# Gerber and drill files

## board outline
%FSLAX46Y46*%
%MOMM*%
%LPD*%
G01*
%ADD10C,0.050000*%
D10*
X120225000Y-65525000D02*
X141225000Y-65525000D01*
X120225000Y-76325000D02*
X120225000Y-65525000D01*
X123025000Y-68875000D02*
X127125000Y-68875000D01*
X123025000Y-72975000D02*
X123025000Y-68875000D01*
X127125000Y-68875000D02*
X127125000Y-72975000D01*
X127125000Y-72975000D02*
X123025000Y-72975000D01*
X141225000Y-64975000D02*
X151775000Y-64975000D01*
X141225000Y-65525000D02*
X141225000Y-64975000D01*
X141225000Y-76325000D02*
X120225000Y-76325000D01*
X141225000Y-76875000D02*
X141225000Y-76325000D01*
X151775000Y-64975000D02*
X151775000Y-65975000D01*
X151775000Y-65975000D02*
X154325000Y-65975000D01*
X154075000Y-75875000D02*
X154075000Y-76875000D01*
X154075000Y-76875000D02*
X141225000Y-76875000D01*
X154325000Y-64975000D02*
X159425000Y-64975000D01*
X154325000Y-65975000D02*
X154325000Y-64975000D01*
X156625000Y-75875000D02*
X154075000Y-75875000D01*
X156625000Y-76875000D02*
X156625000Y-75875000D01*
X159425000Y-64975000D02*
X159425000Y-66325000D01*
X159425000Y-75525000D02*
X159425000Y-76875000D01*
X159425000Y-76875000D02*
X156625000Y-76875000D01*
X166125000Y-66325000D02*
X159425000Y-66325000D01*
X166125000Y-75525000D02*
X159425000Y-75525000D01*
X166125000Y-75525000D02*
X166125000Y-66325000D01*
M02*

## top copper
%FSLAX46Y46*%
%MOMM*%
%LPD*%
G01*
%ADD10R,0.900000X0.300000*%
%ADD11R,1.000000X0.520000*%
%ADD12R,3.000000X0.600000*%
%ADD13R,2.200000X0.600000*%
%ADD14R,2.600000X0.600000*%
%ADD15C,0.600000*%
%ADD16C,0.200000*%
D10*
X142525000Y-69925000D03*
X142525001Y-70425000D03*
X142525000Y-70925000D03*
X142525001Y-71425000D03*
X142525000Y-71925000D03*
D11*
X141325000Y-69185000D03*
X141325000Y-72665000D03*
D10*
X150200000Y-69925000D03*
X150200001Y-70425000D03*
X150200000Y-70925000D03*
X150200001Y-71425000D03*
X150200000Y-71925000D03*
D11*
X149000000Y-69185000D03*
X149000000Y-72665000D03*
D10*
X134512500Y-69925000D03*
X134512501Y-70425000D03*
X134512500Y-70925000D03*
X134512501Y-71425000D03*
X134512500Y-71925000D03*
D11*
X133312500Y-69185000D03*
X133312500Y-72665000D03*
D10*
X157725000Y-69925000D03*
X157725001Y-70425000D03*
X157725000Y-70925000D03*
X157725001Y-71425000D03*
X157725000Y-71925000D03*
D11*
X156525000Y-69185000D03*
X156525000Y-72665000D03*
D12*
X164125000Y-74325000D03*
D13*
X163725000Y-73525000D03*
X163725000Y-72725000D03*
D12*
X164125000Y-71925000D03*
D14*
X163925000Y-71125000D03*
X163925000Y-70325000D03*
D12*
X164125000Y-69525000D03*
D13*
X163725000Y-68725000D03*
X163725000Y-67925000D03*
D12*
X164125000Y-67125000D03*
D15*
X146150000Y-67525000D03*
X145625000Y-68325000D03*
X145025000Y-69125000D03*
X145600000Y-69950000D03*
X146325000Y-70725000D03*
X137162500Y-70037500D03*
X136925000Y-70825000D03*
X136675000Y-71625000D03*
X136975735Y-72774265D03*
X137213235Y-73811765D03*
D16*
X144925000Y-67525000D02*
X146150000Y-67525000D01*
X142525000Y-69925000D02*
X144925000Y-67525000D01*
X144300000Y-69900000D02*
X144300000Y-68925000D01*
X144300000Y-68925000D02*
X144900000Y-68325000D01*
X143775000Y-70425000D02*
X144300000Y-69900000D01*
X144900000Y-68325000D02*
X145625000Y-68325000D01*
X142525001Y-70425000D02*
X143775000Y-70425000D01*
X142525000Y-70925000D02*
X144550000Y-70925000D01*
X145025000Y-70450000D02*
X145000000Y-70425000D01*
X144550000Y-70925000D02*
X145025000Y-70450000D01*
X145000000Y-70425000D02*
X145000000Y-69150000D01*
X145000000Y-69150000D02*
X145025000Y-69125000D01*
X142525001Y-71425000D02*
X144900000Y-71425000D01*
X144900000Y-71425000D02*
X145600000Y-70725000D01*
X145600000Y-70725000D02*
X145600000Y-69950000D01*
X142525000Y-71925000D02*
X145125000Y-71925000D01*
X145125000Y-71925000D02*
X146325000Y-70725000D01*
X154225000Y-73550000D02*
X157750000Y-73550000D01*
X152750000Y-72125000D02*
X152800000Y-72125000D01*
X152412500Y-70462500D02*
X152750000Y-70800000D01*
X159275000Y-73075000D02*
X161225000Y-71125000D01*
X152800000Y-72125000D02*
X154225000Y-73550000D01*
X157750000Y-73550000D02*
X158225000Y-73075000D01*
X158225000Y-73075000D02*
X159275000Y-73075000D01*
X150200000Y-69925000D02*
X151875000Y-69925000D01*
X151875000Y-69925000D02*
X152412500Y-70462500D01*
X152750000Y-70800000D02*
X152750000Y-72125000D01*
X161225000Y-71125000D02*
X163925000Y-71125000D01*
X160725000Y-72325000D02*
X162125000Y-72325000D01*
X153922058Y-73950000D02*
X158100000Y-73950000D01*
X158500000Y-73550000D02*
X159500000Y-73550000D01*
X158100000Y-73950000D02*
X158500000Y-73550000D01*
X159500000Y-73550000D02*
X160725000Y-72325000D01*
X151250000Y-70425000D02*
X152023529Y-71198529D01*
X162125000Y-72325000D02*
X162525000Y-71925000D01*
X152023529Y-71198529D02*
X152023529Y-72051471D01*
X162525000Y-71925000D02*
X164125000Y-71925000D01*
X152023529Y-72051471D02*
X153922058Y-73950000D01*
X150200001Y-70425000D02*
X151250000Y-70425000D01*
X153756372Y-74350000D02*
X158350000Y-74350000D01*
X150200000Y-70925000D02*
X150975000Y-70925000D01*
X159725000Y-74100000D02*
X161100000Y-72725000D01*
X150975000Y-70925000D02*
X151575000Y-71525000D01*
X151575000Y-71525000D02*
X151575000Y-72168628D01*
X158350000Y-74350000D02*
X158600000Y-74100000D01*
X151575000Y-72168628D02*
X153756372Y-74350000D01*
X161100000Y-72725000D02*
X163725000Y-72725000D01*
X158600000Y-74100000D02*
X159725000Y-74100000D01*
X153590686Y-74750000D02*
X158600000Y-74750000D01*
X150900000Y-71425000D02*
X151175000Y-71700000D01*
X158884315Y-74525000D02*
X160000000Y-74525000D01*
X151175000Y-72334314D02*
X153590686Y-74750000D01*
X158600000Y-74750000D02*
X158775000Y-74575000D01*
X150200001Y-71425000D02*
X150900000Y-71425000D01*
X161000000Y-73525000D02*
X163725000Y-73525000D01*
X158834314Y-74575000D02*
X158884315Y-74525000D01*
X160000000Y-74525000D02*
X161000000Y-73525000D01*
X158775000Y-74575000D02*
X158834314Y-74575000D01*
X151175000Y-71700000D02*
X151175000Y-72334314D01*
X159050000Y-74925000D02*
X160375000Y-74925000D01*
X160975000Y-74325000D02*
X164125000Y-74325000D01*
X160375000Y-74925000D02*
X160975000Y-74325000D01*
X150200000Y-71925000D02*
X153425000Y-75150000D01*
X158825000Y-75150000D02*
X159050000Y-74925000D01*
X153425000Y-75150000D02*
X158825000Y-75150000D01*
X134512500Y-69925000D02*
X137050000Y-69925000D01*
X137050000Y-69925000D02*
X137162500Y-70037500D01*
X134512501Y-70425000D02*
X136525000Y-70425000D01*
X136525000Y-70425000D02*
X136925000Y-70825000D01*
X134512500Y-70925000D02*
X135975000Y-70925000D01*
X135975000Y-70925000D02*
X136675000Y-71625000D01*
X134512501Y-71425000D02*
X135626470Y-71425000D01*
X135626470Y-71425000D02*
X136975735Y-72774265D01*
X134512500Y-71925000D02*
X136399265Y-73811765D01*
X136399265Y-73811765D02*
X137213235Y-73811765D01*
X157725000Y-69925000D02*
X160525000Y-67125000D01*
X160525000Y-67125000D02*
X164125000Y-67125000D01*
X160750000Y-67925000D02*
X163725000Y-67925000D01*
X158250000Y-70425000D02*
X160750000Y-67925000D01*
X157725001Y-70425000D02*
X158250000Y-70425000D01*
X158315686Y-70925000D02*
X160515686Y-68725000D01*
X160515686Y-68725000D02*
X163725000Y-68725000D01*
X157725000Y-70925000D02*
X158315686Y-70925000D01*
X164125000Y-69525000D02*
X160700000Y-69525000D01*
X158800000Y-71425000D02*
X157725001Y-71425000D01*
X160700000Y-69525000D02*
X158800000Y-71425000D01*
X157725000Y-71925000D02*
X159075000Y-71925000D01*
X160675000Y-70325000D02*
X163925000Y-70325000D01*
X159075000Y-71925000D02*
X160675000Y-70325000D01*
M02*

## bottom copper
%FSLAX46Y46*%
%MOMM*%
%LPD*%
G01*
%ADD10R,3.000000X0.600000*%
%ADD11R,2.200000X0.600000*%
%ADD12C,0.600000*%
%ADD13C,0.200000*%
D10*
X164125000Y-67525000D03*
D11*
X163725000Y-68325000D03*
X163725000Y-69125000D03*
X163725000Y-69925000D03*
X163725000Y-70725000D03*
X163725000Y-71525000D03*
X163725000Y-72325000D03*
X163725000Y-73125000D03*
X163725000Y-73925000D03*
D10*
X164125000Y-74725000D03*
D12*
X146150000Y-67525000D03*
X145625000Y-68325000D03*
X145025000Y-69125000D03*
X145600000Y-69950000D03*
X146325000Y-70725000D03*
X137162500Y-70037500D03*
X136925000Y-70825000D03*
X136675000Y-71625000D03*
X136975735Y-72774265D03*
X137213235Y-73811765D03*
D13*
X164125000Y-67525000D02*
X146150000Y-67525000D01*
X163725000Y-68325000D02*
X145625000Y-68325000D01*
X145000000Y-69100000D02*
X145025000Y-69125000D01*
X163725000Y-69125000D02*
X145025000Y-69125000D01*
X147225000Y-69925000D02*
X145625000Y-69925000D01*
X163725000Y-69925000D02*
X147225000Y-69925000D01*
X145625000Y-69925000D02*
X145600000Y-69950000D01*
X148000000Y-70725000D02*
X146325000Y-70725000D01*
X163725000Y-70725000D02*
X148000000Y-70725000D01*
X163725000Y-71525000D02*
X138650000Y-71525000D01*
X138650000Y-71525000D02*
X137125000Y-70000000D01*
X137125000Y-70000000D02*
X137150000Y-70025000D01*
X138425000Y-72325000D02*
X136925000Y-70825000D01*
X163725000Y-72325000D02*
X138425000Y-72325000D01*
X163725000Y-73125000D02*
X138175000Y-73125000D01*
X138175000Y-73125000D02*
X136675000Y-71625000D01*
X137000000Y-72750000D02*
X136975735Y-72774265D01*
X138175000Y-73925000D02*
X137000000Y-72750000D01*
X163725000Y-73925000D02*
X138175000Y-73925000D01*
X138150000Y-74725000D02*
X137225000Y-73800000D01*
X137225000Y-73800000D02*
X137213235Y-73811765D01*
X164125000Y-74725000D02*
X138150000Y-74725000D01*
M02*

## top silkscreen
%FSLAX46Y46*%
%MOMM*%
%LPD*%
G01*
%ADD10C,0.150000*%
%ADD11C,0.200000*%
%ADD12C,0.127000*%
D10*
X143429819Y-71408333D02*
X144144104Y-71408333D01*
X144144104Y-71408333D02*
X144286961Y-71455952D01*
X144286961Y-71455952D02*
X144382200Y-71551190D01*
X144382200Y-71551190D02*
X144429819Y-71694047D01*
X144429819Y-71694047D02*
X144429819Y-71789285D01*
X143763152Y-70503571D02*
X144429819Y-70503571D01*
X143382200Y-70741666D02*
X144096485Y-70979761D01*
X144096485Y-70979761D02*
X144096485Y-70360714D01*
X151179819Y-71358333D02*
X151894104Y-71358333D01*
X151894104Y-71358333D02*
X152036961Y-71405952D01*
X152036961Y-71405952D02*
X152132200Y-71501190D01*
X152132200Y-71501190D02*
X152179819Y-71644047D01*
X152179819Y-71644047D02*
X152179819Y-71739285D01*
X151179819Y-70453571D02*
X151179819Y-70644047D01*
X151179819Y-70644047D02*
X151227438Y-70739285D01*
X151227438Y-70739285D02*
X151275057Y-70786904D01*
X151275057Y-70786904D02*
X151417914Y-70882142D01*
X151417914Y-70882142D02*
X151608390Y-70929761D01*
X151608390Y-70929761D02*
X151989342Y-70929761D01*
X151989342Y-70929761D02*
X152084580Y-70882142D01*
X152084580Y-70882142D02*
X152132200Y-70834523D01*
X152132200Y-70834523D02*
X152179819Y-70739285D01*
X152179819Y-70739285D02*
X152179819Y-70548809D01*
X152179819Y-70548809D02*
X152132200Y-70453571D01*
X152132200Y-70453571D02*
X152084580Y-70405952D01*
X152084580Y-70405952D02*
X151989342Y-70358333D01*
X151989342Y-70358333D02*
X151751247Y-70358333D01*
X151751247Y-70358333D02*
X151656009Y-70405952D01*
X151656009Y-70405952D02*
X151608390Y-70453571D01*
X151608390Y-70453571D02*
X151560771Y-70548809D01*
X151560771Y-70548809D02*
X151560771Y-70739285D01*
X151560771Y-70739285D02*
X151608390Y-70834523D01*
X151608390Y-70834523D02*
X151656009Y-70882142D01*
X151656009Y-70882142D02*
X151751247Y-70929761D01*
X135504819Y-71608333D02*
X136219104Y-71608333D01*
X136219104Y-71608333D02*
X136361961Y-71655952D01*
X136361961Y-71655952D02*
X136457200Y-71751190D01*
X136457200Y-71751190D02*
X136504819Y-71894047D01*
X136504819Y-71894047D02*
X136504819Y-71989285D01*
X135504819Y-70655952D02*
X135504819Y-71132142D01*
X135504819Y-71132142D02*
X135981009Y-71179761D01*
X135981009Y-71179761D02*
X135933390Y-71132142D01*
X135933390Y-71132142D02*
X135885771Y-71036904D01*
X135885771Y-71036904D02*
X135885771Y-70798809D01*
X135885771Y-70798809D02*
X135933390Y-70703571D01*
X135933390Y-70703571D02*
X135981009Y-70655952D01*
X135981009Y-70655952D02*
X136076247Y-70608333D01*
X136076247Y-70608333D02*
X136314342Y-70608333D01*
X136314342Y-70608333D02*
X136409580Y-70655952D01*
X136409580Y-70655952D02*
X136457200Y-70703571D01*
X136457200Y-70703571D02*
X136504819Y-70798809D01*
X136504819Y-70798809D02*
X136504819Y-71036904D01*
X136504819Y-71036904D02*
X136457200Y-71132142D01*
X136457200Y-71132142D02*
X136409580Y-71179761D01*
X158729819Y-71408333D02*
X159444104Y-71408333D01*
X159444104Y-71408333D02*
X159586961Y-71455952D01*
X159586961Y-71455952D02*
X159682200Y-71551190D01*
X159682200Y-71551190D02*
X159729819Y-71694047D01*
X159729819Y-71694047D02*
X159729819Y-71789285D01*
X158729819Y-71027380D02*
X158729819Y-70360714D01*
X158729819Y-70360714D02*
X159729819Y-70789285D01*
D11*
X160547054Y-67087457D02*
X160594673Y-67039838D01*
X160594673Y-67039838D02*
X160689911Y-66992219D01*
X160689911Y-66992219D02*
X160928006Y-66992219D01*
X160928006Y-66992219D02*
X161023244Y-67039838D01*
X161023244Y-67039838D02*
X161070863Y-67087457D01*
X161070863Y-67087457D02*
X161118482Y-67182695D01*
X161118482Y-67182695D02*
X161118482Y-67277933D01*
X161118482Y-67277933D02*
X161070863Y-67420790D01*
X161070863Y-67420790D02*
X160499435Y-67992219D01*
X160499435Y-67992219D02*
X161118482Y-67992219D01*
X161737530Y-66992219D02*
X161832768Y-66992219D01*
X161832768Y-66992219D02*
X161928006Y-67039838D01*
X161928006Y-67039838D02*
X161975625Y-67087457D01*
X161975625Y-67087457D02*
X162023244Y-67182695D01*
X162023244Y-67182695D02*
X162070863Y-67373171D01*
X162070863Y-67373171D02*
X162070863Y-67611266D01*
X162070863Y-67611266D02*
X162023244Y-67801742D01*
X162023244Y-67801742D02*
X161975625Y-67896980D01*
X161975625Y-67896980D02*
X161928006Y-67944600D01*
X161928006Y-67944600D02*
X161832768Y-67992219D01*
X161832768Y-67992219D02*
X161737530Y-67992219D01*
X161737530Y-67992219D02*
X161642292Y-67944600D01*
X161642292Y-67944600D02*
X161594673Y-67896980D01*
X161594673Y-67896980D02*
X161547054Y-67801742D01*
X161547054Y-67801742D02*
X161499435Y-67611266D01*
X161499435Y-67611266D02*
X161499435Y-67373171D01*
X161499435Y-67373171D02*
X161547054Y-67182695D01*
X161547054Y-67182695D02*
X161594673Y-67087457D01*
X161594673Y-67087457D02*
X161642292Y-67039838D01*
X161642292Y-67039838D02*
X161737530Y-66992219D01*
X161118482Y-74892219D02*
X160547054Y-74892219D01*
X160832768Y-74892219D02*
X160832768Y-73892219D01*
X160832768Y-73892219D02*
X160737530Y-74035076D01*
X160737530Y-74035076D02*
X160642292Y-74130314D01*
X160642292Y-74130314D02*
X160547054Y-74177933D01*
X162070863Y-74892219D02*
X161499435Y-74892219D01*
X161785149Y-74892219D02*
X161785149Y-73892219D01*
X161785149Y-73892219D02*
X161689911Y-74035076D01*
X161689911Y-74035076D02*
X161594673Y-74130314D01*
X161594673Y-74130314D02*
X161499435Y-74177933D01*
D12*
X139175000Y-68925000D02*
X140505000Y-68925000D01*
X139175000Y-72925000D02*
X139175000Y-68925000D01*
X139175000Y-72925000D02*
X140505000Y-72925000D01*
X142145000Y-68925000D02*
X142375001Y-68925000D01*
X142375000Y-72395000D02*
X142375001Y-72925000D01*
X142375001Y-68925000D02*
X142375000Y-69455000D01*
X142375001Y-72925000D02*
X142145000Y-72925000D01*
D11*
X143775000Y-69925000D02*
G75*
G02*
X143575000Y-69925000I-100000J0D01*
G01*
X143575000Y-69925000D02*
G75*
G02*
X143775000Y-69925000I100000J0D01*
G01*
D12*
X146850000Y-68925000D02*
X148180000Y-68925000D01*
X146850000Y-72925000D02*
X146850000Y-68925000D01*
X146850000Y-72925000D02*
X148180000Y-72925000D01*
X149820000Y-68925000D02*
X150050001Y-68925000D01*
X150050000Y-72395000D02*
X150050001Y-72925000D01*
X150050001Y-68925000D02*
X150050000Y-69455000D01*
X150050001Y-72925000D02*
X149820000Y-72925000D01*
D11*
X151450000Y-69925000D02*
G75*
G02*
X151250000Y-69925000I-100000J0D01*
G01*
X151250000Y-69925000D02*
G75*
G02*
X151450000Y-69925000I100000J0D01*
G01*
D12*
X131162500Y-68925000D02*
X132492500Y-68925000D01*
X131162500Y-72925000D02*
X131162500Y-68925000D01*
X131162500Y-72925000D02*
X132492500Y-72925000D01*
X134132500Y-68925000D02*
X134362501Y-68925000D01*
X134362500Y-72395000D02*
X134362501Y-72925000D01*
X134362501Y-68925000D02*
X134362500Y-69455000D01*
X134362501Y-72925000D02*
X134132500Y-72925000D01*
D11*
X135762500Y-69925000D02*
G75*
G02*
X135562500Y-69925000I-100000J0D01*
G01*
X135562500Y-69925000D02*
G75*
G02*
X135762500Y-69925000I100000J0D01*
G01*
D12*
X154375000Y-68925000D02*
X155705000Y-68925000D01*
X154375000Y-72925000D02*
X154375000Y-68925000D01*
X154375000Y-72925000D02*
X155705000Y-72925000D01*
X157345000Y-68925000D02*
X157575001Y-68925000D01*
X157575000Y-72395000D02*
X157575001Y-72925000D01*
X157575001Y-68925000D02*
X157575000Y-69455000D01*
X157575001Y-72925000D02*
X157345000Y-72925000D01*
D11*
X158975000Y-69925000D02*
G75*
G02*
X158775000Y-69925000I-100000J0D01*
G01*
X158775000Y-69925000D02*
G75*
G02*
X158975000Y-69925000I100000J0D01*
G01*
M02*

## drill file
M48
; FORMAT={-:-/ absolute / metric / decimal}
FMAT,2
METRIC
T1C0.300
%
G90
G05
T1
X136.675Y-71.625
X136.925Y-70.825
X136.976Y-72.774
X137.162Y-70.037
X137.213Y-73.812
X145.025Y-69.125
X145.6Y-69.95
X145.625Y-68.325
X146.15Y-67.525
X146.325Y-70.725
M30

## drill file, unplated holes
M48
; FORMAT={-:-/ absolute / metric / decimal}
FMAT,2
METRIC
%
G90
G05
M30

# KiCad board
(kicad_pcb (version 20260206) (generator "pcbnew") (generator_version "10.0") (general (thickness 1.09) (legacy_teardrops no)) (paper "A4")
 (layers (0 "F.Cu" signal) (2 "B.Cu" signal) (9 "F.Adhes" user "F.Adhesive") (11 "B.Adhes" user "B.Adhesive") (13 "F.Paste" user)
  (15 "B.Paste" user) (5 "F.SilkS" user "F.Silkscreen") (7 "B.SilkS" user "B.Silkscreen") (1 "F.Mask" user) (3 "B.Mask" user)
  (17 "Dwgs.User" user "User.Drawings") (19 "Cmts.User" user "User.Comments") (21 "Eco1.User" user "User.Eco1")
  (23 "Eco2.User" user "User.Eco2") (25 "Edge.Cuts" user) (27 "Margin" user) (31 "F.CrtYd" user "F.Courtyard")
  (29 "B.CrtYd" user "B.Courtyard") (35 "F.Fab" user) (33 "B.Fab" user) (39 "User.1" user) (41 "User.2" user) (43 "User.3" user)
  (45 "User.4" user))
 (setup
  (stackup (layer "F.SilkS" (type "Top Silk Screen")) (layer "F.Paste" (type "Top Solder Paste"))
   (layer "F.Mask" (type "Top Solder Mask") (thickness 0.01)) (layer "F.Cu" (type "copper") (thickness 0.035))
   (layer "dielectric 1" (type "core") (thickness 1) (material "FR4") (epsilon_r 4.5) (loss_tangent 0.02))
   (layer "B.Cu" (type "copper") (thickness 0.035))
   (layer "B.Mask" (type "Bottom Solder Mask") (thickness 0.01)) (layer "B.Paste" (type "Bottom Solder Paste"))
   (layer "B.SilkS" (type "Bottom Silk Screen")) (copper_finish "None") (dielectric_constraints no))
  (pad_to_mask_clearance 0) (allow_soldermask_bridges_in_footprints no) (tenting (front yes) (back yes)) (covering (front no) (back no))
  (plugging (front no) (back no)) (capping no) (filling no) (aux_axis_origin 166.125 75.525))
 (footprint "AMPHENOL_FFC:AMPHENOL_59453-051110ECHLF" (layer "F.Cu") (at 141.325 70.925 -90)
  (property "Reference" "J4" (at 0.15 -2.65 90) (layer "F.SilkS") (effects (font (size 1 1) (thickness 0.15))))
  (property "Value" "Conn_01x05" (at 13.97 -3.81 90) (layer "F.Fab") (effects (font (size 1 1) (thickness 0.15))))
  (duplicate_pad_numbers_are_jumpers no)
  (fp_line (start -2 2.15) (end -2 0.82) (stroke (width 0.127) (type solid)) (layer "F.SilkS"))
  (fp_line (start 2 2.15) (end -2 2.15) (stroke (width 0.127) (type solid)) (layer "F.SilkS"))
  (fp_line (start 2 2.15) (end 2 0.82) (stroke (width 0.127) (type solid)) (layer "F.SilkS"))
  (fp_line (start -2 -0.82) (end -2 -1.050001) (stroke (width 0.127) (type solid)) (layer "F.SilkS"))
  (fp_line (start 1.47 -1.05) (end 2 -1.050001) (stroke (width 0.127) (type solid)) (layer "F.SilkS"))
  (fp_line (start -2 -1.050001) (end -1.47 -1.05) (stroke (width 0.127) (type solid)) (layer "F.SilkS"))
  (fp_line (start 2 -1.050001) (end 2 -0.82) (stroke (width 0.127) (type solid)) (layer "F.SilkS"))
  (fp_circle (center -1 -2.35) (end -0.9 -2.35) (stroke (width 0.2) (type solid)) (fill no) (layer "F.SilkS"))
  (pad "1" smd rect (at -1 -1.2 270) (size 0.3 0.9) (layers "F.Cu" "F.Mask" "F.Paste") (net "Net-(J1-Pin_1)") (solder_mask_margin 0.102))
  (pad "2" smd rect (at -0.5 -1.200001 270) (size 0.3 0.9) (layers "F.Cu" "F.Mask" "F.Paste") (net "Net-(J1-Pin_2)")
   (solder_mask_margin 0.102))
  (pad "3" smd rect (at 0 -1.2 270) (size 0.3 0.9) (layers "F.Cu" "F.Mask" "F.Paste") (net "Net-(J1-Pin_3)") (solder_mask_margin 0.102))
  (pad "4" smd rect (at 0.5 -1.200001 270) (size 0.3 0.9) (layers "F.Cu" "F.Mask" "F.Paste") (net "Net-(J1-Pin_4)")
   (solder_mask_margin 0.102))
  (pad "5" smd rect (at 1 -1.2 270) (size 0.3 0.9) (layers "F.Cu" "F.Mask" "F.Paste") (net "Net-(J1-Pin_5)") (solder_mask_margin 0.102))
  (pad "S1" smd rect (at -1.74 0 270) (size 0.52 1) (layers "F.Cu" "F.Mask" "F.Paste") (solder_mask_margin 0.102))
  (pad "S2" smd rect (at 1.74 0 270) (size 0.52 1) (layers "F.Cu" "F.Mask" "F.Paste") (solder_mask_margin 0.102)))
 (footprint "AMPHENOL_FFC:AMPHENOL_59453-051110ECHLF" (layer "F.Cu") (at 149 70.925 -90)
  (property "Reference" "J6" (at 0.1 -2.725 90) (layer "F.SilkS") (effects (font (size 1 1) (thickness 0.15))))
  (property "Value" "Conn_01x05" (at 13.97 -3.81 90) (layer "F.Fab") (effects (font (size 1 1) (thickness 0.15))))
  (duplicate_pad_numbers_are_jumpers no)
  (fp_line (start -2 2.15) (end -2 0.82) (stroke (width 0.127) (type solid)) (layer "F.SilkS"))
  (fp_line (start 2 2.15) (end -2 2.15) (stroke (width 0.127) (type solid)) (layer "F.SilkS"))
  (fp_line (start 2 2.15) (end 2 0.82) (stroke (width 0.127) (type solid)) (layer "F.SilkS"))
  (fp_line (start -2 -0.82) (end -2 -1.050001) (stroke (width 0.127) (type solid)) (layer "F.SilkS"))
  (fp_line (start 1.47 -1.05) (end 2 -1.050001) (stroke (width 0.127) (type solid)) (layer "F.SilkS"))
  (fp_line (start -2 -1.050001) (end -1.47 -1.05) (stroke (width 0.127) (type solid)) (layer "F.SilkS"))
  (fp_line (start 2 -1.050001) (end 2 -0.82) (stroke (width 0.127) (type solid)) (layer "F.SilkS"))
  (fp_circle (center -1 -2.35) (end -0.9 -2.35) (stroke (width 0.2) (type solid)) (fill no) (layer "F.SilkS"))
  (pad "1" smd rect (at -1 -1.2 270) (size 0.3 0.9) (layers "F.Cu" "F.Mask" "F.Paste") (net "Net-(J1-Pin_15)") (solder_mask_margin 0.102))
  (pad "2" smd rect (at -0.5 -1.200001 270) (size 0.3 0.9) (layers "F.Cu" "F.Mask" "F.Paste") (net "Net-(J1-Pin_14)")
   (solder_mask_margin 0.102))
  (pad "3" smd rect (at 0 -1.2 270) (size 0.3 0.9) (layers "F.Cu" "F.Mask" "F.Paste") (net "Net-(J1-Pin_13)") (solder_mask_margin 0.102))
  (pad "4" smd rect (at 0.5 -1.200001 270) (size 0.3 0.9) (layers "F.Cu" "F.Mask" "F.Paste") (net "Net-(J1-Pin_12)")
   (solder_mask_margin 0.102))
  (pad "5" smd rect (at 1 -1.2 270) (size 0.3 0.9) (layers "F.Cu" "F.Mask" "F.Paste") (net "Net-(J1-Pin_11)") (solder_mask_margin 0.102))
  (pad "S1" smd rect (at -1.74 0 270) (size 0.52 1) (layers "F.Cu" "F.Mask" "F.Paste") (solder_mask_margin 0.102))
  (pad "S2" smd rect (at 1.74 0 270) (size 0.52 1) (layers "F.Cu" "F.Mask" "F.Paste") (solder_mask_margin 0.102)))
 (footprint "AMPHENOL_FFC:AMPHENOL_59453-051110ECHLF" (layer "F.Cu") (at 133.3125 70.925 -90)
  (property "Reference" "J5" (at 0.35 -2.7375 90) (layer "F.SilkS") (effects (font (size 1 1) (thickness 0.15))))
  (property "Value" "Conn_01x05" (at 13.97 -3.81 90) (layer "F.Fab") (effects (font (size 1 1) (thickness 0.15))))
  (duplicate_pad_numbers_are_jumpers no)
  (fp_line (start -2 2.15) (end -2 0.82) (stroke (width 0.127) (type solid)) (layer "F.SilkS"))
  (fp_line (start 2 2.15) (end -2 2.15) (stroke (width 0.127) (type solid)) (layer "F.SilkS"))
  (fp_line (start 2 2.15) (end 2 0.82) (stroke (width 0.127) (type solid)) (layer "F.SilkS"))
  (fp_line (start -2 -0.82) (end -2 -1.050001) (stroke (width 0.127) (type solid)) (layer "F.SilkS"))
  (fp_line (start 1.47 -1.05) (end 2 -1.050001) (stroke (width 0.127) (type solid)) (layer "F.SilkS"))
  (fp_line (start -2 -1.050001) (end -1.47 -1.05) (stroke (width 0.127) (type solid)) (layer "F.SilkS"))
  (fp_line (start 2 -1.050001) (end 2 -0.82) (stroke (width 0.127) (type solid)) (layer "F.SilkS"))
  (fp_circle (center -1 -2.35) (end -0.9 -2.35) (stroke (width 0.2) (type solid)) (fill no) (layer "F.SilkS"))
  (pad "1" smd rect (at -1 -1.2 270) (size 0.3 0.9) (layers "F.Cu" "F.Mask" "F.Paste") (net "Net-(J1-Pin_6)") (solder_mask_margin 0.102))
  (pad "2" smd rect (at -0.5 -1.200001 270) (size 0.3 0.9) (layers "F.Cu" "F.Mask" "F.Paste") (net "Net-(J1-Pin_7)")
   (solder_mask_margin 0.102))
  (pad "3" smd rect (at 0 -1.2 270) (size 0.3 0.9) (layers "F.Cu" "F.Mask" "F.Paste") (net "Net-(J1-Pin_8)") (solder_mask_margin 0.102))
  (pad "4" smd rect (at 0.5 -1.200001 270) (size 0.3 0.9) (layers "F.Cu" "F.Mask" "F.Paste") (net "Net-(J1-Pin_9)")
   (solder_mask_margin 0.102))
  (pad "5" smd rect (at 1 -1.2 270) (size 0.3 0.9) (layers "F.Cu" "F.Mask" "F.Paste") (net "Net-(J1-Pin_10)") (solder_mask_margin 0.102))
  (pad "S1" smd rect (at -1.74 0 270) (size 0.52 1) (layers "F.Cu" "F.Mask" "F.Paste") (solder_mask_margin 0.102))
  (pad "S2" smd rect (at 1.74 0 270) (size 0.52 1) (layers "F.Cu" "F.Mask" "F.Paste") (solder_mask_margin 0.102)))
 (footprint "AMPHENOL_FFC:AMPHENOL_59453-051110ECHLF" (layer "F.Cu") (at 156.525 70.925 -90)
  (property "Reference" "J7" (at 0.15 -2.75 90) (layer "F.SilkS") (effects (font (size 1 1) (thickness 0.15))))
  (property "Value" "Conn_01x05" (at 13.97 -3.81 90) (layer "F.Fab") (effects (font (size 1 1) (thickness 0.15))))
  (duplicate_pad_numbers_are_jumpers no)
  (fp_line (start -2 2.15) (end -2 0.82) (stroke (width 0.127) (type solid)) (layer "F.SilkS"))
  (fp_line (start 2 2.15) (end -2 2.15) (stroke (width 0.127) (type solid)) (layer "F.SilkS"))
  (fp_line (start 2 2.15) (end 2 0.82) (stroke (width 0.127) (type solid)) (layer "F.SilkS"))
  (fp_line (start -2 -0.82) (end -2 -1.050001) (stroke (width 0.127) (type solid)) (layer "F.SilkS"))
  (fp_line (start 1.47 -1.05) (end 2 -1.050001) (stroke (width 0.127) (type solid)) (layer "F.SilkS"))
  (fp_line (start -2 -1.050001) (end -1.47 -1.05) (stroke (width 0.127) (type solid)) (layer "F.SilkS"))
  (fp_line (start 2 -1.050001) (end 2 -0.82) (stroke (width 0.127) (type solid)) (layer "F.SilkS"))
  (fp_circle (center -1 -2.35) (end -0.9 -2.35) (stroke (width 0.2) (type solid)) (fill no) (layer "F.SilkS"))
  (pad "1" smd rect (at -1 -1.2 270) (size 0.3 0.9) (layers "F.Cu" "F.Mask" "F.Paste") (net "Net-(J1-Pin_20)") (solder_mask_margin 0.102))
  (pad "2" smd rect (at -0.5 -1.200001 270) (size 0.3 0.9) (layers "F.Cu" "F.Mask" "F.Paste") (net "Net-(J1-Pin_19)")
   (solder_mask_margin 0.102))
  (pad "3" smd rect (at 0 -1.2 270) (size 0.3 0.9) (layers "F.Cu" "F.Mask" "F.Paste") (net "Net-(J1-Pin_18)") (solder_mask_margin 0.102))
  (pad "4" smd rect (at 0.5 -1.200001 270) (size 0.3 0.9) (layers "F.Cu" "F.Mask" "F.Paste") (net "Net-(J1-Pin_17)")
   (solder_mask_margin 0.102))
  (pad "5" smd rect (at 1 -1.2 270) (size 0.3 0.9) (layers "F.Cu" "F.Mask" "F.Paste") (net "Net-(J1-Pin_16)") (solder_mask_margin 0.102))
  (pad "S1" smd rect (at -1.74 0 270) (size 0.52 1) (layers "F.Cu" "F.Mask" "F.Paste") (solder_mask_margin 0.102))
  (pad "S2" smd rect (at 1.74 0 270) (size 0.52 1) (layers "F.Cu" "F.Mask" "F.Paste") (solder_mask_margin 0.102)))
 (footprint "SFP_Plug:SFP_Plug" (layer "F.Cu") (at 162.625 70.925)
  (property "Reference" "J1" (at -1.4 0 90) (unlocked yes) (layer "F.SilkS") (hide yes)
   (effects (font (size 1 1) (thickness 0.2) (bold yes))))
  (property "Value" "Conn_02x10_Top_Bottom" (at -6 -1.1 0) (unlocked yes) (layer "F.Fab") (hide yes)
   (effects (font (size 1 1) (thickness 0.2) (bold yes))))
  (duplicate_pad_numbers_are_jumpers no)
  (fp_line (start -42.4 -5.4) (end -21.4 -5.4) (stroke (width 0.05) (type default)) (layer "Edge.Cuts"))
  (fp_line (start -42.4 5.4) (end -42.4 -5.4) (stroke (width 0.05) (type default)) (layer "Edge.Cuts"))
  (fp_line (start -39.6 -2.05) (end -35.5 -2.05) (stroke (width 0.05) (type default)) (layer "Edge.Cuts"))
  (fp_line (start -39.6 2.05) (end -39.6 -2.05) (stroke (width 0.05) (type default)) (layer "Edge.Cuts"))
  (fp_line (start -35.5 -2.05) (end -35.5 2.05) (stroke (width 0.05) (type default)) (layer "Edge.Cuts"))
  (fp_line (start -35.5 2.05) (end -39.6 2.05) (stroke (width 0.05) (type default)) (layer "Edge.Cuts"))
  (fp_line (start -21.4 -5.95) (end -10.85 -5.95) (stroke (width 0.05) (type default)) (layer "Edge.Cuts"))
  (fp_line (start -21.4 -5.4) (end -21.4 -5.95) (stroke (width 0.05) (type default)) (layer "Edge.Cuts"))
  (fp_line (start -21.4 5.4) (end -42.4 5.4) (stroke (width 0.05) (type default)) (layer "Edge.Cuts"))
  (fp_line (start -21.4 5.95) (end -21.4 5.4) (stroke (width 0.05) (type default)) (layer "Edge.Cuts"))
  (fp_line (start -10.85 -5.95) (end -10.85 -4.95) (stroke (width 0.05) (type default)) (layer "Edge.Cuts"))
  (fp_line (start -10.85 -4.95) (end -8.3 -4.95) (stroke (width 0.05) (type default)) (layer "Edge.Cuts"))
  (fp_line (start -8.55 4.95) (end -8.55 5.95) (stroke (width 0.05) (type default)) (layer "Edge.Cuts"))
  (fp_line (start -8.55 5.95) (end -21.4 5.95) (stroke (width 0.05) (type default)) (layer "Edge.Cuts"))
  (fp_line (start -8.3 -5.95) (end -3.2 -5.95) (stroke (width 0.05) (type default)) (layer "Edge.Cuts"))
  (fp_line (start -8.3 -4.95) (end -8.3 -5.95) (stroke (width 0.05) (type default)) (layer "Edge.Cuts"))
  (fp_line (start -6 4.95) (end -8.55 4.95) (stroke (width 0.05) (type default)) (layer "Edge.Cuts"))
  (fp_line (start -6 5.95) (end -6 4.95) (stroke (width 0.05) (type default)) (layer "Edge.Cuts"))
  (fp_line (start -3.2 -5.95) (end -3.2 -4.6) (stroke (width 0.05) (type default)) (layer "Edge.Cuts"))
  (fp_line (start -3.2 4.6) (end -3.2 5.95) (stroke (width 0.05) (type default)) (layer "Edge.Cuts"))
  (fp_line (start -3.2 5.95) (end -6 5.95) (stroke (width 0.05) (type default)) (layer "Edge.Cuts"))
  (fp_line (start 3.5 -4.6) (end -3.2 -4.6) (stroke (width 0.05) (type solid)) (layer "Edge.Cuts"))
  (fp_line (start 3.5 4.6) (end -3.2 4.6) (stroke (width 0.05) (type solid)) (layer "Edge.Cuts"))
  (fp_line (start 3.5 4.6) (end 3.5 -4.6) (stroke (width 0.05) (type default)) (layer "Edge.Cuts"))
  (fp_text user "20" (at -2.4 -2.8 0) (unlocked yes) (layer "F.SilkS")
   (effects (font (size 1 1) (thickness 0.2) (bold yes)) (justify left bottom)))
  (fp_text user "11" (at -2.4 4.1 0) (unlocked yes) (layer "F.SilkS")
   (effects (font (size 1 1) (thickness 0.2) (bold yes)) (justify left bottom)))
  (pad "1" smd rect (at 1.5 -3.4) (size 3 0.6) (layers "B.Cu" "B.Mask") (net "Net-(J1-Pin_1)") (thermal_bridge_angle 45))
  (pad "2" smd rect (at 1.1 -2.6) (size 2.2 0.6) (layers "B.Cu" "B.Mask") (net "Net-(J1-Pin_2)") (thermal_bridge_angle 45))
  (pad "3" smd rect (at 1.1 -1.8) (size 2.2 0.6) (layers "B.Cu" "B.Mask") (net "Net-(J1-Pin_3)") (thermal_bridge_angle 45))
  (pad "4" smd rect (at 1.1 -1) (size 2.2 0.6) (layers "B.Cu" "B.Mask") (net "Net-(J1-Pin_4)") (thermal_bridge_angle 45))
  (pad "5" smd rect (at 1.1 -0.2) (size 2.2 0.6) (layers "B.Cu" "B.Mask") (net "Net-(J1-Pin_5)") (thermal_bridge_angle 45))
  (pad "6" smd rect (at 1.1 0.6) (size 2.2 0.6) (layers "B.Cu" "B.Mask") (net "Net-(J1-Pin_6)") (thermal_bridge_angle 45))
  (pad "7" smd rect (at 1.1 1.4) (size 2.2 0.6) (layers "B.Cu" "B.Mask") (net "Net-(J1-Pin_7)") (thermal_bridge_angle 45))
  (pad "8" smd rect (at 1.1 2.2) (size 2.2 0.6) (layers "B.Cu" "B.Mask") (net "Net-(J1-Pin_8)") (thermal_bridge_angle 45))
  (pad "9" smd rect (at 1.1 3) (size 2.2 0.6) (layers "B.Cu" "B.Mask") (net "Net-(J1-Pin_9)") (thermal_bridge_angle 45))
  (pad "10" smd rect (at 1.5 3.8) (size 3 0.6) (layers "B.Cu" "B.Mask") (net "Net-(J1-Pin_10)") (thermal_bridge_angle 45))
  (pad "11" smd rect (at 1.5 3.4) (size 3 0.6) (layers "F.Cu" "F.Mask") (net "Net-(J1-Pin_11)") (thermal_bridge_angle 45))
  (pad "12" smd rect (at 1.1 2.6) (size 2.2 0.6) (layers "F.Cu" "F.Mask") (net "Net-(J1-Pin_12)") (thermal_bridge_angle 45))
  (pad "13" smd rect (at 1.1 1.8) (size 2.2 0.6) (layers "F.Cu" "F.Mask") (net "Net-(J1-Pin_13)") (thermal_bridge_angle 45))
  (pad "14" smd rect (at 1.5 1) (size 3 0.6) (layers "F.Cu" "F.Mask") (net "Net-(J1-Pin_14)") (thermal_bridge_angle 45))
  (pad "15" smd rect (at 1.3 0.2) (size 2.6 0.6) (layers "F.Cu" "F.Mask") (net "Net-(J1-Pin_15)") (thermal_bridge_angle 45))
  (pad "16" smd rect (at 1.3 -0.6) (size 2.6 0.6) (layers "F.Cu" "F.Mask") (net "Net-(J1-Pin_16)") (thermal_bridge_angle 45))
  (pad "17" smd rect (at 1.5 -1.4) (size 3 0.6) (layers "F.Cu" "F.Mask") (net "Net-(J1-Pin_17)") (thermal_bridge_angle 45))
  (pad "18" smd rect (at 1.1 -2.2) (size 2.2 0.6) (layers "F.Cu" "F.Mask") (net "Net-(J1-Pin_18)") (thermal_bridge_angle 45))
  (pad "19" smd rect (at 1.1 -3) (size 2.2 0.6) (layers "F.Cu" "F.Mask") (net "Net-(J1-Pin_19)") (thermal_bridge_angle 45))
  (pad "20" smd rect (at 1.5 -3.8) (size 3 0.6) (layers "F.Cu" "F.Mask") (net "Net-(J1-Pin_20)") (thermal_bridge_angle 45)))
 (segment (start 144.925 67.525) (end 146.15 67.525) (width 0.2) (layer "F.Cu") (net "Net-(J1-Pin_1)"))
 (segment (start 142.525 69.925) (end 144.925 67.525) (width 0.2) (layer "F.Cu") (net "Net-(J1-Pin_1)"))
 (via (at 146.15 67.525) (size 0.6) (drill 0.3) (layers "F.Cu" "B.Cu") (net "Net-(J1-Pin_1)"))
 (segment (start 164.125 67.525) (end 146.15 67.525) (width 0.2) (layer "B.Cu") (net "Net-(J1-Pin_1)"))
 (segment (start 144.3 69.9) (end 144.3 68.925) (width 0.2) (layer "F.Cu") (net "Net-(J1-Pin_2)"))
 (segment (start 144.3 68.925) (end 144.9 68.325) (width 0.2) (layer "F.Cu") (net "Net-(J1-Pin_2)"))
 (segment (start 143.775 70.425) (end 144.3 69.9) (width 0.2) (layer "F.Cu") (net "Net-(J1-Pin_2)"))
 (segment (start 144.9 68.325) (end 145.625 68.325) (width 0.2) (layer "F.Cu") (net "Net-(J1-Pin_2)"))
 (segment (start 142.525001 70.425) (end 143.775 70.425) (width 0.2) (layer "F.Cu") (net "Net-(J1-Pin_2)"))
 (via (at 145.625 68.325) (size 0.6) (drill 0.3) (layers "F.Cu" "B.Cu") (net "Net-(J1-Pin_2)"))
 (segment (start 163.725 68.325) (end 145.625 68.325) (width 0.2) (layer "B.Cu") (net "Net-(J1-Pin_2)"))
 (segment (start 142.525 70.925) (end 144.55 70.925) (width 0.2) (layer "F.Cu") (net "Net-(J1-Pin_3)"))
 (segment (start 145.025 70.45) (end 145 70.425) (width 0.2) (layer "F.Cu") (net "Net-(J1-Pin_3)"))
 (segment (start 144.55 70.925) (end 145.025 70.45) (width 0.2) (layer "F.Cu") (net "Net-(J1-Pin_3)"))
 (segment (start 145 70.425) (end 145 69.15) (width 0.2) (layer "F.Cu") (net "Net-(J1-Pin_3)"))
 (segment (start 145 69.15) (end 145.025 69.125) (width 0.2) (layer "F.Cu") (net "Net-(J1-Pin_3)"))
 (via (at 145.025 69.125) (size 0.6) (drill 0.3) (layers "F.Cu" "B.Cu") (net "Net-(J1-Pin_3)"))
 (segment (start 145 69.1) (end 145.025 69.125) (width 0.2) (layer "B.Cu") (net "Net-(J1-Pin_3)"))
 (segment (start 163.725 69.125) (end 145.025 69.125) (width 0.2) (layer "B.Cu") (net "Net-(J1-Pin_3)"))
 (segment (start 142.525001 71.425) (end 144.9 71.425) (width 0.2) (layer "F.Cu") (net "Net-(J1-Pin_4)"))
 (segment (start 144.9 71.425) (end 145.6 70.725) (width 0.2) (layer "F.Cu") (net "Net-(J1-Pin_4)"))
 (segment (start 145.6 70.725) (end 145.6 69.95) (width 0.2) (layer "F.Cu") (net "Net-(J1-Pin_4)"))
 (via (at 145.6 69.95) (size 0.6) (drill 0.3) (layers "F.Cu" "B.Cu") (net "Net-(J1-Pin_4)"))
 (segment (start 147.225 69.925) (end 145.625 69.925) (width 0.2) (layer "B.Cu") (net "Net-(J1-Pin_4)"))
 (segment (start 163.725 69.925) (end 147.225 69.925) (width 0.2) (layer "B.Cu") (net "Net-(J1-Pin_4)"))
 (segment (start 145.625 69.925) (end 145.6 69.95) (width 0.2) (layer "B.Cu") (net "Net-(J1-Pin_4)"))
 (segment (start 142.525 71.925) (end 145.125 71.925) (width 0.2) (layer "F.Cu") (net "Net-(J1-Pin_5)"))
 (segment (start 145.125 71.925) (end 146.325 70.725) (width 0.2) (layer "F.Cu") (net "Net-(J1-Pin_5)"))
 (via (at 146.325 70.725) (size 0.6) (drill 0.3) (layers "F.Cu" "B.Cu") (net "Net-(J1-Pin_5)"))
 (segment (start 148 70.725) (end 146.325 70.725) (width 0.2) (layer "B.Cu") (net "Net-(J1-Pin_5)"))
 (segment (start 163.725 70.725) (end 148 70.725) (width 0.2) (layer "B.Cu") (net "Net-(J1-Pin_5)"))
 (segment (start 154.225 73.55) (end 157.75 73.55) (width 0.2) (layer "F.Cu") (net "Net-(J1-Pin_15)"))
 (segment (start 152.75 72.125) (end 152.8 72.125) (width 0.2) (layer "F.Cu") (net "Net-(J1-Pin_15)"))
 (segment (start 152.4125 70.4625) (end 152.75 70.8) (width 0.2) (layer "F.Cu") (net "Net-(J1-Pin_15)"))
 (segment (start 159.275 73.075) (end 161.225 71.125) (width 0.2) (layer "F.Cu") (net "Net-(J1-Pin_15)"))
 (segment (start 152.8 72.125) (end 154.225 73.55) (width 0.2) (layer "F.Cu") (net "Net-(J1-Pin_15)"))
 (segment (start 157.75 73.55) (end 158.225 73.075) (width 0.2) (layer "F.Cu") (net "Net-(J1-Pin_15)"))
 (segment (start 158.225 73.075) (end 159.275 73.075) (width 0.2) (layer "F.Cu") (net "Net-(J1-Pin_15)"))
 (segment (start 150.2 69.925) (end 151.875 69.925) (width 0.2) (layer "F.Cu") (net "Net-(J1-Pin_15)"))
 (segment (start 151.875 69.925) (end 152.4125 70.4625) (width 0.2) (layer "F.Cu") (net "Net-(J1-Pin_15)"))
 (segment (start 152.75 70.8) (end 152.75 72.125) (width 0.2) (layer "F.Cu") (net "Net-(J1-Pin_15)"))
 (segment (start 161.225 71.125) (end 163.925 71.125) (width 0.2) (layer "F.Cu") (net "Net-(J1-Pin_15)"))
 (segment (start 160.725 72.325) (end 162.125 72.325) (width 0.2) (layer "F.Cu") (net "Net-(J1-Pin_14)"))
 (segment (start 153.922058 73.95) (end 158.1 73.95) (width 0.2) (layer "F.Cu") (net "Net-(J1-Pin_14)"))
 (segment (start 158.5 73.55) (end 159.5 73.55) (width 0.2) (layer "F.Cu") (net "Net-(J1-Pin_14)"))
 (segment (start 158.1 73.95) (end 158.5 73.55) (width 0.2) (layer "F.Cu") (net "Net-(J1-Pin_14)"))
 (segment (start 159.5 73.55) (end 160.725 72.325) (width 0.2) (layer "F.Cu") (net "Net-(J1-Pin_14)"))
 (segment (start 151.25 70.425) (end 152.023529 71.198529) (width 0.2) (layer "F.Cu") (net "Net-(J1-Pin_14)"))
 (segment (start 162.125 72.325) (end 162.525 71.925) (width 0.2) (layer "F.Cu") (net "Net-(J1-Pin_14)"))
 (segment (start 152.023529 71.198529) (end 152.023529 72.051471) (width 0.2) (layer "F.Cu") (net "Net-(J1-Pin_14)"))
 (segment (start 162.525 71.925) (end 164.125 71.925) (width 0.2) (layer "F.Cu") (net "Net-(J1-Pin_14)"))
 (segment (start 152.023529 72.051471) (end 153.922058 73.95) (width 0.2) (layer "F.Cu") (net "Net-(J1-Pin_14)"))
 (segment (start 150.200001 70.425) (end 151.25 70.425) (width 0.2) (layer "F.Cu") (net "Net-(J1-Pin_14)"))
 (segment (start 153.756372 74.35) (end 158.35 74.35) (width 0.2) (layer "F.Cu") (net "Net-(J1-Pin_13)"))
 (segment (start 150.2 70.925) (end 150.975 70.925) (width 0.2) (layer "F.Cu") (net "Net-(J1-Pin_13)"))
 (segment (start 159.725 74.1) (end 161.1 72.725) (width 0.2) (layer "F.Cu") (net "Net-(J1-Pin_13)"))
 (segment (start 150.975 70.925) (end 151.575 71.525) (width 0.2) (layer "F.Cu") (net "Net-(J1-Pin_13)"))
 (segment (start 151.575 71.525) (end 151.575 72.168628) (width 0.2) (layer "F.Cu") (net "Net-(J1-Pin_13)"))
 (segment (start 158.35 74.35) (end 158.6 74.1) (width 0.2) (layer "F.Cu") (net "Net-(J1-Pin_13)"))
 (segment (start 151.575 72.168628) (end 153.756372 74.35) (width 0.2) (layer "F.Cu") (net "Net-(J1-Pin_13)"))
 (segment (start 161.1 72.725) (end 163.725 72.725) (width 0.2) (layer "F.Cu") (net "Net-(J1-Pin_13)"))
 (segment (start 158.6 74.1) (end 159.725 74.1) (width 0.2) (layer "F.Cu") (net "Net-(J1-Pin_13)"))
 (segment (start 153.590686 74.75) (end 158.6 74.75) (width 0.2) (layer "F.Cu") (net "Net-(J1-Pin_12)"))
 (segment (start 150.9 71.425) (end 151.175 71.7) (width 0.2) (layer "F.Cu") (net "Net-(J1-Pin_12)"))
 (segment (start 158.884315 74.525) (end 160 74.525) (width 0.2) (layer "F.Cu") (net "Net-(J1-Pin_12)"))
 (segment (start 151.175 72.334314) (end 153.590686 74.75) (width 0.2) (layer "F.Cu") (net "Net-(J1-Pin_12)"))
 (segment (start 158.6 74.75) (end 158.775 74.575) (width 0.2) (layer "F.Cu") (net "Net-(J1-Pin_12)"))
 (segment (start 150.200001 71.425) (end 150.9 71.425) (width 0.2) (layer "F.Cu") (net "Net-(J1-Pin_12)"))
 (segment (start 161 73.525) (end 163.725 73.525) (width 0.2) (layer "F.Cu") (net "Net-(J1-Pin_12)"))
 (segment (start 158.834314 74.575) (end 158.884315 74.525) (width 0.2) (layer "F.Cu") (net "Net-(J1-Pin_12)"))
 (segment (start 160 74.525) (end 161 73.525) (width 0.2) (layer "F.Cu") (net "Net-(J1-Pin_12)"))
 (segment (start 158.775 74.575) (end 158.834314 74.575) (width 0.2) (layer "F.Cu") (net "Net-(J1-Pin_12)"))
 (segment (start 151.175 71.7) (end 151.175 72.334314) (width 0.2) (layer "F.Cu") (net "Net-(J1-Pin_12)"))
 (segment (start 159.05 74.925) (end 160.375 74.925) (width 0.2) (layer "F.Cu") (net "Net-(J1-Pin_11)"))
 (segment (start 160.975 74.325) (end 164.125 74.325) (width 0.2) (layer "F.Cu") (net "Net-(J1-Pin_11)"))
 (segment (start 160.375 74.925) (end 160.975 74.325) (width 0.2) (layer "F.Cu") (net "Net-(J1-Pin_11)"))
 (segment (start 150.2 71.925) (end 153.425 75.15) (width 0.2) (layer "F.Cu") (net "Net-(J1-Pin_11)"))
 (segment (start 158.825 75.15) (end 159.05 74.925) (width 0.2) (layer "F.Cu") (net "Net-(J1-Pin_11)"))
 (segment (start 153.425 75.15) (end 158.825 75.15) (width 0.2) (layer "F.Cu") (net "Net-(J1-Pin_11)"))
 (segment (start 134.5125 69.925) (end 137.05 69.925) (width 0.2) (layer "F.Cu") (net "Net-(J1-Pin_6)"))
 (segment (start 137.05 69.925) (end 137.1625 70.0375) (width 0.2) (layer "F.Cu") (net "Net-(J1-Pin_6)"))
 (via (at 137.1625 70.0375) (size 0.6) (drill 0.3) (layers "F.Cu" "B.Cu") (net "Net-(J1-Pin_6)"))
 (segment (start 163.725 71.525) (end 138.65 71.525) (width 0.2) (layer "B.Cu") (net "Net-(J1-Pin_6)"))
 (segment (start 138.65 71.525) (end 137.125 70) (width 0.2) (layer "B.Cu") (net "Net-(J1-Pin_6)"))
 (segment (start 137.125 70) (end 137.15 70.025) (width 0.2) (layer "B.Cu") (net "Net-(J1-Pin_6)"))
 (segment (start 134.512501 70.425) (end 136.525 70.425) (width 0.2) (layer "F.Cu") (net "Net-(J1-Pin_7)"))
 (segment (start 136.525 70.425) (end 136.925 70.825) (width 0.2) (layer "F.Cu") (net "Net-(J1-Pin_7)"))
 (via (at 136.925 70.825) (size 0.6) (drill 0.3) (layers "F.Cu" "B.Cu") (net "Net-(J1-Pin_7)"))
 (segment (start 138.425 72.325) (end 136.925 70.825) (width 0.2) (layer "B.Cu") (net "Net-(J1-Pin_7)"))
 (segment (start 163.725 72.325) (end 138.425 72.325) (width 0.2) (layer "B.Cu") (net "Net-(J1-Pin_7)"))
 (segment (start 134.5125 70.925) (end 135.975 70.925) (width 0.2) (layer "F.Cu") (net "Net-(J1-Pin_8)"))
 (segment (start 135.975 70.925) (end 136.675 71.625) (width 0.2) (layer "F.Cu") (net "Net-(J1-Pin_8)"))
 (via (at 136.675 71.625) (size 0.6) (drill 0.3) (layers "F.Cu" "B.Cu") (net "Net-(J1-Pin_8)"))
 (segment (start 163.725 73.125) (end 138.175 73.125) (width 0.2) (layer "B.Cu") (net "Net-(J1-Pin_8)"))
 (segment (start 138.175 73.125) (end 136.675 71.625) (width 0.2) (layer "B.Cu") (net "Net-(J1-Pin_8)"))
 (segment (start 134.512501 71.425) (end 135.62647 71.425) (width 0.2) (layer "F.Cu") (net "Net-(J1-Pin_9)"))
 (segment (start 135.62647 71.425) (end 136.975735 72.774265) (width 0.2) (layer "F.Cu") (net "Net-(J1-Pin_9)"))
 (via (at 136.975735 72.774265) (size 0.6) (drill 0.3) (layers "F.Cu" "B.Cu") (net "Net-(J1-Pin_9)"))
 (segment (start 137 72.75) (end 136.975735 72.774265) (width 0.2) (layer "B.Cu") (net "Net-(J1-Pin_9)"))
 (segment (start 138.175 73.925) (end 137 72.75) (width 0.2) (layer "B.Cu") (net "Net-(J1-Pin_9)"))
 (segment (start 163.725 73.925) (end 138.175 73.925) (width 0.2) (layer "B.Cu") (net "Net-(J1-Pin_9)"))
 (segment (start 134.5125 71.925) (end 136.399265 73.811765) (width 0.2) (layer "F.Cu") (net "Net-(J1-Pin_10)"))
 (segment (start 136.399265 73.811765) (end 137.213235 73.811765) (width 0.2) (layer "F.Cu") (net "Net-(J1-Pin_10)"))
 (via (at 137.213235 73.811765) (size 0.6) (drill 0.3) (layers "F.Cu" "B.Cu") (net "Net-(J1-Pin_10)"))
 (segment (start 138.15 74.725) (end 137.225 73.8) (width 0.2) (layer "B.Cu") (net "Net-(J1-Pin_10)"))
 (segment (start 137.225 73.8) (end 137.213235 73.811765) (width 0.2) (layer "B.Cu") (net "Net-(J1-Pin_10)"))
 (segment (start 164.125 74.725) (end 138.15 74.725) (width 0.2) (layer "B.Cu") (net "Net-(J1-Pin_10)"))
 (segment (start 157.725 69.925) (end 160.525 67.125) (width 0.2) (layer "F.Cu") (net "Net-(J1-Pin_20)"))
 (segment (start 160.525 67.125) (end 164.125 67.125) (width 0.2) (layer "F.Cu") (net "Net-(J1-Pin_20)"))
 (segment (start 160.75 67.925) (end 163.725 67.925) (width 0.2) (layer "F.Cu") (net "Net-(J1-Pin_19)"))
 (segment (start 158.25 70.425) (end 160.75 67.925) (width 0.2) (layer "F.Cu") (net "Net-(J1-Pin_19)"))
 (segment (start 157.725001 70.425) (end 158.25 70.425) (width 0.2) (layer "F.Cu") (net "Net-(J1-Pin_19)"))
 (segment (start 158.315686 70.925) (end 160.515686 68.725) (width 0.2) (layer "F.Cu") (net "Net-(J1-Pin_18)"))
 (segment (start 160.515686 68.725) (end 163.725 68.725) (width 0.2) (layer "F.Cu") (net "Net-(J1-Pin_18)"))
 (segment (start 157.725 70.925) (end 158.315686 70.925) (width 0.2) (layer "F.Cu") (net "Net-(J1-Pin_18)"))
 (segment (start 164.125 69.525) (end 160.7 69.525) (width 0.2) (layer "F.Cu") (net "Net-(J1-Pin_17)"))
 (segment (start 158.8 71.425) (end 157.725001 71.425) (width 0.2) (layer "F.Cu") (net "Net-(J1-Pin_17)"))
 (segment (start 160.7 69.525) (end 158.8 71.425) (width 0.2) (layer "F.Cu") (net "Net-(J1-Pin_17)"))
 (segment (start 157.725 71.925) (end 159.075 71.925) (width 0.2) (layer "F.Cu") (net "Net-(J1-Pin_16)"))
 (segment (start 160.675 70.325) (end 163.925 70.325) (width 0.2) (layer "F.Cu") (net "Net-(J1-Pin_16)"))
 (segment (start 159.075 71.925) (end 160.675 70.325) (width 0.2) (layer "F.Cu") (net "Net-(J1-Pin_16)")))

